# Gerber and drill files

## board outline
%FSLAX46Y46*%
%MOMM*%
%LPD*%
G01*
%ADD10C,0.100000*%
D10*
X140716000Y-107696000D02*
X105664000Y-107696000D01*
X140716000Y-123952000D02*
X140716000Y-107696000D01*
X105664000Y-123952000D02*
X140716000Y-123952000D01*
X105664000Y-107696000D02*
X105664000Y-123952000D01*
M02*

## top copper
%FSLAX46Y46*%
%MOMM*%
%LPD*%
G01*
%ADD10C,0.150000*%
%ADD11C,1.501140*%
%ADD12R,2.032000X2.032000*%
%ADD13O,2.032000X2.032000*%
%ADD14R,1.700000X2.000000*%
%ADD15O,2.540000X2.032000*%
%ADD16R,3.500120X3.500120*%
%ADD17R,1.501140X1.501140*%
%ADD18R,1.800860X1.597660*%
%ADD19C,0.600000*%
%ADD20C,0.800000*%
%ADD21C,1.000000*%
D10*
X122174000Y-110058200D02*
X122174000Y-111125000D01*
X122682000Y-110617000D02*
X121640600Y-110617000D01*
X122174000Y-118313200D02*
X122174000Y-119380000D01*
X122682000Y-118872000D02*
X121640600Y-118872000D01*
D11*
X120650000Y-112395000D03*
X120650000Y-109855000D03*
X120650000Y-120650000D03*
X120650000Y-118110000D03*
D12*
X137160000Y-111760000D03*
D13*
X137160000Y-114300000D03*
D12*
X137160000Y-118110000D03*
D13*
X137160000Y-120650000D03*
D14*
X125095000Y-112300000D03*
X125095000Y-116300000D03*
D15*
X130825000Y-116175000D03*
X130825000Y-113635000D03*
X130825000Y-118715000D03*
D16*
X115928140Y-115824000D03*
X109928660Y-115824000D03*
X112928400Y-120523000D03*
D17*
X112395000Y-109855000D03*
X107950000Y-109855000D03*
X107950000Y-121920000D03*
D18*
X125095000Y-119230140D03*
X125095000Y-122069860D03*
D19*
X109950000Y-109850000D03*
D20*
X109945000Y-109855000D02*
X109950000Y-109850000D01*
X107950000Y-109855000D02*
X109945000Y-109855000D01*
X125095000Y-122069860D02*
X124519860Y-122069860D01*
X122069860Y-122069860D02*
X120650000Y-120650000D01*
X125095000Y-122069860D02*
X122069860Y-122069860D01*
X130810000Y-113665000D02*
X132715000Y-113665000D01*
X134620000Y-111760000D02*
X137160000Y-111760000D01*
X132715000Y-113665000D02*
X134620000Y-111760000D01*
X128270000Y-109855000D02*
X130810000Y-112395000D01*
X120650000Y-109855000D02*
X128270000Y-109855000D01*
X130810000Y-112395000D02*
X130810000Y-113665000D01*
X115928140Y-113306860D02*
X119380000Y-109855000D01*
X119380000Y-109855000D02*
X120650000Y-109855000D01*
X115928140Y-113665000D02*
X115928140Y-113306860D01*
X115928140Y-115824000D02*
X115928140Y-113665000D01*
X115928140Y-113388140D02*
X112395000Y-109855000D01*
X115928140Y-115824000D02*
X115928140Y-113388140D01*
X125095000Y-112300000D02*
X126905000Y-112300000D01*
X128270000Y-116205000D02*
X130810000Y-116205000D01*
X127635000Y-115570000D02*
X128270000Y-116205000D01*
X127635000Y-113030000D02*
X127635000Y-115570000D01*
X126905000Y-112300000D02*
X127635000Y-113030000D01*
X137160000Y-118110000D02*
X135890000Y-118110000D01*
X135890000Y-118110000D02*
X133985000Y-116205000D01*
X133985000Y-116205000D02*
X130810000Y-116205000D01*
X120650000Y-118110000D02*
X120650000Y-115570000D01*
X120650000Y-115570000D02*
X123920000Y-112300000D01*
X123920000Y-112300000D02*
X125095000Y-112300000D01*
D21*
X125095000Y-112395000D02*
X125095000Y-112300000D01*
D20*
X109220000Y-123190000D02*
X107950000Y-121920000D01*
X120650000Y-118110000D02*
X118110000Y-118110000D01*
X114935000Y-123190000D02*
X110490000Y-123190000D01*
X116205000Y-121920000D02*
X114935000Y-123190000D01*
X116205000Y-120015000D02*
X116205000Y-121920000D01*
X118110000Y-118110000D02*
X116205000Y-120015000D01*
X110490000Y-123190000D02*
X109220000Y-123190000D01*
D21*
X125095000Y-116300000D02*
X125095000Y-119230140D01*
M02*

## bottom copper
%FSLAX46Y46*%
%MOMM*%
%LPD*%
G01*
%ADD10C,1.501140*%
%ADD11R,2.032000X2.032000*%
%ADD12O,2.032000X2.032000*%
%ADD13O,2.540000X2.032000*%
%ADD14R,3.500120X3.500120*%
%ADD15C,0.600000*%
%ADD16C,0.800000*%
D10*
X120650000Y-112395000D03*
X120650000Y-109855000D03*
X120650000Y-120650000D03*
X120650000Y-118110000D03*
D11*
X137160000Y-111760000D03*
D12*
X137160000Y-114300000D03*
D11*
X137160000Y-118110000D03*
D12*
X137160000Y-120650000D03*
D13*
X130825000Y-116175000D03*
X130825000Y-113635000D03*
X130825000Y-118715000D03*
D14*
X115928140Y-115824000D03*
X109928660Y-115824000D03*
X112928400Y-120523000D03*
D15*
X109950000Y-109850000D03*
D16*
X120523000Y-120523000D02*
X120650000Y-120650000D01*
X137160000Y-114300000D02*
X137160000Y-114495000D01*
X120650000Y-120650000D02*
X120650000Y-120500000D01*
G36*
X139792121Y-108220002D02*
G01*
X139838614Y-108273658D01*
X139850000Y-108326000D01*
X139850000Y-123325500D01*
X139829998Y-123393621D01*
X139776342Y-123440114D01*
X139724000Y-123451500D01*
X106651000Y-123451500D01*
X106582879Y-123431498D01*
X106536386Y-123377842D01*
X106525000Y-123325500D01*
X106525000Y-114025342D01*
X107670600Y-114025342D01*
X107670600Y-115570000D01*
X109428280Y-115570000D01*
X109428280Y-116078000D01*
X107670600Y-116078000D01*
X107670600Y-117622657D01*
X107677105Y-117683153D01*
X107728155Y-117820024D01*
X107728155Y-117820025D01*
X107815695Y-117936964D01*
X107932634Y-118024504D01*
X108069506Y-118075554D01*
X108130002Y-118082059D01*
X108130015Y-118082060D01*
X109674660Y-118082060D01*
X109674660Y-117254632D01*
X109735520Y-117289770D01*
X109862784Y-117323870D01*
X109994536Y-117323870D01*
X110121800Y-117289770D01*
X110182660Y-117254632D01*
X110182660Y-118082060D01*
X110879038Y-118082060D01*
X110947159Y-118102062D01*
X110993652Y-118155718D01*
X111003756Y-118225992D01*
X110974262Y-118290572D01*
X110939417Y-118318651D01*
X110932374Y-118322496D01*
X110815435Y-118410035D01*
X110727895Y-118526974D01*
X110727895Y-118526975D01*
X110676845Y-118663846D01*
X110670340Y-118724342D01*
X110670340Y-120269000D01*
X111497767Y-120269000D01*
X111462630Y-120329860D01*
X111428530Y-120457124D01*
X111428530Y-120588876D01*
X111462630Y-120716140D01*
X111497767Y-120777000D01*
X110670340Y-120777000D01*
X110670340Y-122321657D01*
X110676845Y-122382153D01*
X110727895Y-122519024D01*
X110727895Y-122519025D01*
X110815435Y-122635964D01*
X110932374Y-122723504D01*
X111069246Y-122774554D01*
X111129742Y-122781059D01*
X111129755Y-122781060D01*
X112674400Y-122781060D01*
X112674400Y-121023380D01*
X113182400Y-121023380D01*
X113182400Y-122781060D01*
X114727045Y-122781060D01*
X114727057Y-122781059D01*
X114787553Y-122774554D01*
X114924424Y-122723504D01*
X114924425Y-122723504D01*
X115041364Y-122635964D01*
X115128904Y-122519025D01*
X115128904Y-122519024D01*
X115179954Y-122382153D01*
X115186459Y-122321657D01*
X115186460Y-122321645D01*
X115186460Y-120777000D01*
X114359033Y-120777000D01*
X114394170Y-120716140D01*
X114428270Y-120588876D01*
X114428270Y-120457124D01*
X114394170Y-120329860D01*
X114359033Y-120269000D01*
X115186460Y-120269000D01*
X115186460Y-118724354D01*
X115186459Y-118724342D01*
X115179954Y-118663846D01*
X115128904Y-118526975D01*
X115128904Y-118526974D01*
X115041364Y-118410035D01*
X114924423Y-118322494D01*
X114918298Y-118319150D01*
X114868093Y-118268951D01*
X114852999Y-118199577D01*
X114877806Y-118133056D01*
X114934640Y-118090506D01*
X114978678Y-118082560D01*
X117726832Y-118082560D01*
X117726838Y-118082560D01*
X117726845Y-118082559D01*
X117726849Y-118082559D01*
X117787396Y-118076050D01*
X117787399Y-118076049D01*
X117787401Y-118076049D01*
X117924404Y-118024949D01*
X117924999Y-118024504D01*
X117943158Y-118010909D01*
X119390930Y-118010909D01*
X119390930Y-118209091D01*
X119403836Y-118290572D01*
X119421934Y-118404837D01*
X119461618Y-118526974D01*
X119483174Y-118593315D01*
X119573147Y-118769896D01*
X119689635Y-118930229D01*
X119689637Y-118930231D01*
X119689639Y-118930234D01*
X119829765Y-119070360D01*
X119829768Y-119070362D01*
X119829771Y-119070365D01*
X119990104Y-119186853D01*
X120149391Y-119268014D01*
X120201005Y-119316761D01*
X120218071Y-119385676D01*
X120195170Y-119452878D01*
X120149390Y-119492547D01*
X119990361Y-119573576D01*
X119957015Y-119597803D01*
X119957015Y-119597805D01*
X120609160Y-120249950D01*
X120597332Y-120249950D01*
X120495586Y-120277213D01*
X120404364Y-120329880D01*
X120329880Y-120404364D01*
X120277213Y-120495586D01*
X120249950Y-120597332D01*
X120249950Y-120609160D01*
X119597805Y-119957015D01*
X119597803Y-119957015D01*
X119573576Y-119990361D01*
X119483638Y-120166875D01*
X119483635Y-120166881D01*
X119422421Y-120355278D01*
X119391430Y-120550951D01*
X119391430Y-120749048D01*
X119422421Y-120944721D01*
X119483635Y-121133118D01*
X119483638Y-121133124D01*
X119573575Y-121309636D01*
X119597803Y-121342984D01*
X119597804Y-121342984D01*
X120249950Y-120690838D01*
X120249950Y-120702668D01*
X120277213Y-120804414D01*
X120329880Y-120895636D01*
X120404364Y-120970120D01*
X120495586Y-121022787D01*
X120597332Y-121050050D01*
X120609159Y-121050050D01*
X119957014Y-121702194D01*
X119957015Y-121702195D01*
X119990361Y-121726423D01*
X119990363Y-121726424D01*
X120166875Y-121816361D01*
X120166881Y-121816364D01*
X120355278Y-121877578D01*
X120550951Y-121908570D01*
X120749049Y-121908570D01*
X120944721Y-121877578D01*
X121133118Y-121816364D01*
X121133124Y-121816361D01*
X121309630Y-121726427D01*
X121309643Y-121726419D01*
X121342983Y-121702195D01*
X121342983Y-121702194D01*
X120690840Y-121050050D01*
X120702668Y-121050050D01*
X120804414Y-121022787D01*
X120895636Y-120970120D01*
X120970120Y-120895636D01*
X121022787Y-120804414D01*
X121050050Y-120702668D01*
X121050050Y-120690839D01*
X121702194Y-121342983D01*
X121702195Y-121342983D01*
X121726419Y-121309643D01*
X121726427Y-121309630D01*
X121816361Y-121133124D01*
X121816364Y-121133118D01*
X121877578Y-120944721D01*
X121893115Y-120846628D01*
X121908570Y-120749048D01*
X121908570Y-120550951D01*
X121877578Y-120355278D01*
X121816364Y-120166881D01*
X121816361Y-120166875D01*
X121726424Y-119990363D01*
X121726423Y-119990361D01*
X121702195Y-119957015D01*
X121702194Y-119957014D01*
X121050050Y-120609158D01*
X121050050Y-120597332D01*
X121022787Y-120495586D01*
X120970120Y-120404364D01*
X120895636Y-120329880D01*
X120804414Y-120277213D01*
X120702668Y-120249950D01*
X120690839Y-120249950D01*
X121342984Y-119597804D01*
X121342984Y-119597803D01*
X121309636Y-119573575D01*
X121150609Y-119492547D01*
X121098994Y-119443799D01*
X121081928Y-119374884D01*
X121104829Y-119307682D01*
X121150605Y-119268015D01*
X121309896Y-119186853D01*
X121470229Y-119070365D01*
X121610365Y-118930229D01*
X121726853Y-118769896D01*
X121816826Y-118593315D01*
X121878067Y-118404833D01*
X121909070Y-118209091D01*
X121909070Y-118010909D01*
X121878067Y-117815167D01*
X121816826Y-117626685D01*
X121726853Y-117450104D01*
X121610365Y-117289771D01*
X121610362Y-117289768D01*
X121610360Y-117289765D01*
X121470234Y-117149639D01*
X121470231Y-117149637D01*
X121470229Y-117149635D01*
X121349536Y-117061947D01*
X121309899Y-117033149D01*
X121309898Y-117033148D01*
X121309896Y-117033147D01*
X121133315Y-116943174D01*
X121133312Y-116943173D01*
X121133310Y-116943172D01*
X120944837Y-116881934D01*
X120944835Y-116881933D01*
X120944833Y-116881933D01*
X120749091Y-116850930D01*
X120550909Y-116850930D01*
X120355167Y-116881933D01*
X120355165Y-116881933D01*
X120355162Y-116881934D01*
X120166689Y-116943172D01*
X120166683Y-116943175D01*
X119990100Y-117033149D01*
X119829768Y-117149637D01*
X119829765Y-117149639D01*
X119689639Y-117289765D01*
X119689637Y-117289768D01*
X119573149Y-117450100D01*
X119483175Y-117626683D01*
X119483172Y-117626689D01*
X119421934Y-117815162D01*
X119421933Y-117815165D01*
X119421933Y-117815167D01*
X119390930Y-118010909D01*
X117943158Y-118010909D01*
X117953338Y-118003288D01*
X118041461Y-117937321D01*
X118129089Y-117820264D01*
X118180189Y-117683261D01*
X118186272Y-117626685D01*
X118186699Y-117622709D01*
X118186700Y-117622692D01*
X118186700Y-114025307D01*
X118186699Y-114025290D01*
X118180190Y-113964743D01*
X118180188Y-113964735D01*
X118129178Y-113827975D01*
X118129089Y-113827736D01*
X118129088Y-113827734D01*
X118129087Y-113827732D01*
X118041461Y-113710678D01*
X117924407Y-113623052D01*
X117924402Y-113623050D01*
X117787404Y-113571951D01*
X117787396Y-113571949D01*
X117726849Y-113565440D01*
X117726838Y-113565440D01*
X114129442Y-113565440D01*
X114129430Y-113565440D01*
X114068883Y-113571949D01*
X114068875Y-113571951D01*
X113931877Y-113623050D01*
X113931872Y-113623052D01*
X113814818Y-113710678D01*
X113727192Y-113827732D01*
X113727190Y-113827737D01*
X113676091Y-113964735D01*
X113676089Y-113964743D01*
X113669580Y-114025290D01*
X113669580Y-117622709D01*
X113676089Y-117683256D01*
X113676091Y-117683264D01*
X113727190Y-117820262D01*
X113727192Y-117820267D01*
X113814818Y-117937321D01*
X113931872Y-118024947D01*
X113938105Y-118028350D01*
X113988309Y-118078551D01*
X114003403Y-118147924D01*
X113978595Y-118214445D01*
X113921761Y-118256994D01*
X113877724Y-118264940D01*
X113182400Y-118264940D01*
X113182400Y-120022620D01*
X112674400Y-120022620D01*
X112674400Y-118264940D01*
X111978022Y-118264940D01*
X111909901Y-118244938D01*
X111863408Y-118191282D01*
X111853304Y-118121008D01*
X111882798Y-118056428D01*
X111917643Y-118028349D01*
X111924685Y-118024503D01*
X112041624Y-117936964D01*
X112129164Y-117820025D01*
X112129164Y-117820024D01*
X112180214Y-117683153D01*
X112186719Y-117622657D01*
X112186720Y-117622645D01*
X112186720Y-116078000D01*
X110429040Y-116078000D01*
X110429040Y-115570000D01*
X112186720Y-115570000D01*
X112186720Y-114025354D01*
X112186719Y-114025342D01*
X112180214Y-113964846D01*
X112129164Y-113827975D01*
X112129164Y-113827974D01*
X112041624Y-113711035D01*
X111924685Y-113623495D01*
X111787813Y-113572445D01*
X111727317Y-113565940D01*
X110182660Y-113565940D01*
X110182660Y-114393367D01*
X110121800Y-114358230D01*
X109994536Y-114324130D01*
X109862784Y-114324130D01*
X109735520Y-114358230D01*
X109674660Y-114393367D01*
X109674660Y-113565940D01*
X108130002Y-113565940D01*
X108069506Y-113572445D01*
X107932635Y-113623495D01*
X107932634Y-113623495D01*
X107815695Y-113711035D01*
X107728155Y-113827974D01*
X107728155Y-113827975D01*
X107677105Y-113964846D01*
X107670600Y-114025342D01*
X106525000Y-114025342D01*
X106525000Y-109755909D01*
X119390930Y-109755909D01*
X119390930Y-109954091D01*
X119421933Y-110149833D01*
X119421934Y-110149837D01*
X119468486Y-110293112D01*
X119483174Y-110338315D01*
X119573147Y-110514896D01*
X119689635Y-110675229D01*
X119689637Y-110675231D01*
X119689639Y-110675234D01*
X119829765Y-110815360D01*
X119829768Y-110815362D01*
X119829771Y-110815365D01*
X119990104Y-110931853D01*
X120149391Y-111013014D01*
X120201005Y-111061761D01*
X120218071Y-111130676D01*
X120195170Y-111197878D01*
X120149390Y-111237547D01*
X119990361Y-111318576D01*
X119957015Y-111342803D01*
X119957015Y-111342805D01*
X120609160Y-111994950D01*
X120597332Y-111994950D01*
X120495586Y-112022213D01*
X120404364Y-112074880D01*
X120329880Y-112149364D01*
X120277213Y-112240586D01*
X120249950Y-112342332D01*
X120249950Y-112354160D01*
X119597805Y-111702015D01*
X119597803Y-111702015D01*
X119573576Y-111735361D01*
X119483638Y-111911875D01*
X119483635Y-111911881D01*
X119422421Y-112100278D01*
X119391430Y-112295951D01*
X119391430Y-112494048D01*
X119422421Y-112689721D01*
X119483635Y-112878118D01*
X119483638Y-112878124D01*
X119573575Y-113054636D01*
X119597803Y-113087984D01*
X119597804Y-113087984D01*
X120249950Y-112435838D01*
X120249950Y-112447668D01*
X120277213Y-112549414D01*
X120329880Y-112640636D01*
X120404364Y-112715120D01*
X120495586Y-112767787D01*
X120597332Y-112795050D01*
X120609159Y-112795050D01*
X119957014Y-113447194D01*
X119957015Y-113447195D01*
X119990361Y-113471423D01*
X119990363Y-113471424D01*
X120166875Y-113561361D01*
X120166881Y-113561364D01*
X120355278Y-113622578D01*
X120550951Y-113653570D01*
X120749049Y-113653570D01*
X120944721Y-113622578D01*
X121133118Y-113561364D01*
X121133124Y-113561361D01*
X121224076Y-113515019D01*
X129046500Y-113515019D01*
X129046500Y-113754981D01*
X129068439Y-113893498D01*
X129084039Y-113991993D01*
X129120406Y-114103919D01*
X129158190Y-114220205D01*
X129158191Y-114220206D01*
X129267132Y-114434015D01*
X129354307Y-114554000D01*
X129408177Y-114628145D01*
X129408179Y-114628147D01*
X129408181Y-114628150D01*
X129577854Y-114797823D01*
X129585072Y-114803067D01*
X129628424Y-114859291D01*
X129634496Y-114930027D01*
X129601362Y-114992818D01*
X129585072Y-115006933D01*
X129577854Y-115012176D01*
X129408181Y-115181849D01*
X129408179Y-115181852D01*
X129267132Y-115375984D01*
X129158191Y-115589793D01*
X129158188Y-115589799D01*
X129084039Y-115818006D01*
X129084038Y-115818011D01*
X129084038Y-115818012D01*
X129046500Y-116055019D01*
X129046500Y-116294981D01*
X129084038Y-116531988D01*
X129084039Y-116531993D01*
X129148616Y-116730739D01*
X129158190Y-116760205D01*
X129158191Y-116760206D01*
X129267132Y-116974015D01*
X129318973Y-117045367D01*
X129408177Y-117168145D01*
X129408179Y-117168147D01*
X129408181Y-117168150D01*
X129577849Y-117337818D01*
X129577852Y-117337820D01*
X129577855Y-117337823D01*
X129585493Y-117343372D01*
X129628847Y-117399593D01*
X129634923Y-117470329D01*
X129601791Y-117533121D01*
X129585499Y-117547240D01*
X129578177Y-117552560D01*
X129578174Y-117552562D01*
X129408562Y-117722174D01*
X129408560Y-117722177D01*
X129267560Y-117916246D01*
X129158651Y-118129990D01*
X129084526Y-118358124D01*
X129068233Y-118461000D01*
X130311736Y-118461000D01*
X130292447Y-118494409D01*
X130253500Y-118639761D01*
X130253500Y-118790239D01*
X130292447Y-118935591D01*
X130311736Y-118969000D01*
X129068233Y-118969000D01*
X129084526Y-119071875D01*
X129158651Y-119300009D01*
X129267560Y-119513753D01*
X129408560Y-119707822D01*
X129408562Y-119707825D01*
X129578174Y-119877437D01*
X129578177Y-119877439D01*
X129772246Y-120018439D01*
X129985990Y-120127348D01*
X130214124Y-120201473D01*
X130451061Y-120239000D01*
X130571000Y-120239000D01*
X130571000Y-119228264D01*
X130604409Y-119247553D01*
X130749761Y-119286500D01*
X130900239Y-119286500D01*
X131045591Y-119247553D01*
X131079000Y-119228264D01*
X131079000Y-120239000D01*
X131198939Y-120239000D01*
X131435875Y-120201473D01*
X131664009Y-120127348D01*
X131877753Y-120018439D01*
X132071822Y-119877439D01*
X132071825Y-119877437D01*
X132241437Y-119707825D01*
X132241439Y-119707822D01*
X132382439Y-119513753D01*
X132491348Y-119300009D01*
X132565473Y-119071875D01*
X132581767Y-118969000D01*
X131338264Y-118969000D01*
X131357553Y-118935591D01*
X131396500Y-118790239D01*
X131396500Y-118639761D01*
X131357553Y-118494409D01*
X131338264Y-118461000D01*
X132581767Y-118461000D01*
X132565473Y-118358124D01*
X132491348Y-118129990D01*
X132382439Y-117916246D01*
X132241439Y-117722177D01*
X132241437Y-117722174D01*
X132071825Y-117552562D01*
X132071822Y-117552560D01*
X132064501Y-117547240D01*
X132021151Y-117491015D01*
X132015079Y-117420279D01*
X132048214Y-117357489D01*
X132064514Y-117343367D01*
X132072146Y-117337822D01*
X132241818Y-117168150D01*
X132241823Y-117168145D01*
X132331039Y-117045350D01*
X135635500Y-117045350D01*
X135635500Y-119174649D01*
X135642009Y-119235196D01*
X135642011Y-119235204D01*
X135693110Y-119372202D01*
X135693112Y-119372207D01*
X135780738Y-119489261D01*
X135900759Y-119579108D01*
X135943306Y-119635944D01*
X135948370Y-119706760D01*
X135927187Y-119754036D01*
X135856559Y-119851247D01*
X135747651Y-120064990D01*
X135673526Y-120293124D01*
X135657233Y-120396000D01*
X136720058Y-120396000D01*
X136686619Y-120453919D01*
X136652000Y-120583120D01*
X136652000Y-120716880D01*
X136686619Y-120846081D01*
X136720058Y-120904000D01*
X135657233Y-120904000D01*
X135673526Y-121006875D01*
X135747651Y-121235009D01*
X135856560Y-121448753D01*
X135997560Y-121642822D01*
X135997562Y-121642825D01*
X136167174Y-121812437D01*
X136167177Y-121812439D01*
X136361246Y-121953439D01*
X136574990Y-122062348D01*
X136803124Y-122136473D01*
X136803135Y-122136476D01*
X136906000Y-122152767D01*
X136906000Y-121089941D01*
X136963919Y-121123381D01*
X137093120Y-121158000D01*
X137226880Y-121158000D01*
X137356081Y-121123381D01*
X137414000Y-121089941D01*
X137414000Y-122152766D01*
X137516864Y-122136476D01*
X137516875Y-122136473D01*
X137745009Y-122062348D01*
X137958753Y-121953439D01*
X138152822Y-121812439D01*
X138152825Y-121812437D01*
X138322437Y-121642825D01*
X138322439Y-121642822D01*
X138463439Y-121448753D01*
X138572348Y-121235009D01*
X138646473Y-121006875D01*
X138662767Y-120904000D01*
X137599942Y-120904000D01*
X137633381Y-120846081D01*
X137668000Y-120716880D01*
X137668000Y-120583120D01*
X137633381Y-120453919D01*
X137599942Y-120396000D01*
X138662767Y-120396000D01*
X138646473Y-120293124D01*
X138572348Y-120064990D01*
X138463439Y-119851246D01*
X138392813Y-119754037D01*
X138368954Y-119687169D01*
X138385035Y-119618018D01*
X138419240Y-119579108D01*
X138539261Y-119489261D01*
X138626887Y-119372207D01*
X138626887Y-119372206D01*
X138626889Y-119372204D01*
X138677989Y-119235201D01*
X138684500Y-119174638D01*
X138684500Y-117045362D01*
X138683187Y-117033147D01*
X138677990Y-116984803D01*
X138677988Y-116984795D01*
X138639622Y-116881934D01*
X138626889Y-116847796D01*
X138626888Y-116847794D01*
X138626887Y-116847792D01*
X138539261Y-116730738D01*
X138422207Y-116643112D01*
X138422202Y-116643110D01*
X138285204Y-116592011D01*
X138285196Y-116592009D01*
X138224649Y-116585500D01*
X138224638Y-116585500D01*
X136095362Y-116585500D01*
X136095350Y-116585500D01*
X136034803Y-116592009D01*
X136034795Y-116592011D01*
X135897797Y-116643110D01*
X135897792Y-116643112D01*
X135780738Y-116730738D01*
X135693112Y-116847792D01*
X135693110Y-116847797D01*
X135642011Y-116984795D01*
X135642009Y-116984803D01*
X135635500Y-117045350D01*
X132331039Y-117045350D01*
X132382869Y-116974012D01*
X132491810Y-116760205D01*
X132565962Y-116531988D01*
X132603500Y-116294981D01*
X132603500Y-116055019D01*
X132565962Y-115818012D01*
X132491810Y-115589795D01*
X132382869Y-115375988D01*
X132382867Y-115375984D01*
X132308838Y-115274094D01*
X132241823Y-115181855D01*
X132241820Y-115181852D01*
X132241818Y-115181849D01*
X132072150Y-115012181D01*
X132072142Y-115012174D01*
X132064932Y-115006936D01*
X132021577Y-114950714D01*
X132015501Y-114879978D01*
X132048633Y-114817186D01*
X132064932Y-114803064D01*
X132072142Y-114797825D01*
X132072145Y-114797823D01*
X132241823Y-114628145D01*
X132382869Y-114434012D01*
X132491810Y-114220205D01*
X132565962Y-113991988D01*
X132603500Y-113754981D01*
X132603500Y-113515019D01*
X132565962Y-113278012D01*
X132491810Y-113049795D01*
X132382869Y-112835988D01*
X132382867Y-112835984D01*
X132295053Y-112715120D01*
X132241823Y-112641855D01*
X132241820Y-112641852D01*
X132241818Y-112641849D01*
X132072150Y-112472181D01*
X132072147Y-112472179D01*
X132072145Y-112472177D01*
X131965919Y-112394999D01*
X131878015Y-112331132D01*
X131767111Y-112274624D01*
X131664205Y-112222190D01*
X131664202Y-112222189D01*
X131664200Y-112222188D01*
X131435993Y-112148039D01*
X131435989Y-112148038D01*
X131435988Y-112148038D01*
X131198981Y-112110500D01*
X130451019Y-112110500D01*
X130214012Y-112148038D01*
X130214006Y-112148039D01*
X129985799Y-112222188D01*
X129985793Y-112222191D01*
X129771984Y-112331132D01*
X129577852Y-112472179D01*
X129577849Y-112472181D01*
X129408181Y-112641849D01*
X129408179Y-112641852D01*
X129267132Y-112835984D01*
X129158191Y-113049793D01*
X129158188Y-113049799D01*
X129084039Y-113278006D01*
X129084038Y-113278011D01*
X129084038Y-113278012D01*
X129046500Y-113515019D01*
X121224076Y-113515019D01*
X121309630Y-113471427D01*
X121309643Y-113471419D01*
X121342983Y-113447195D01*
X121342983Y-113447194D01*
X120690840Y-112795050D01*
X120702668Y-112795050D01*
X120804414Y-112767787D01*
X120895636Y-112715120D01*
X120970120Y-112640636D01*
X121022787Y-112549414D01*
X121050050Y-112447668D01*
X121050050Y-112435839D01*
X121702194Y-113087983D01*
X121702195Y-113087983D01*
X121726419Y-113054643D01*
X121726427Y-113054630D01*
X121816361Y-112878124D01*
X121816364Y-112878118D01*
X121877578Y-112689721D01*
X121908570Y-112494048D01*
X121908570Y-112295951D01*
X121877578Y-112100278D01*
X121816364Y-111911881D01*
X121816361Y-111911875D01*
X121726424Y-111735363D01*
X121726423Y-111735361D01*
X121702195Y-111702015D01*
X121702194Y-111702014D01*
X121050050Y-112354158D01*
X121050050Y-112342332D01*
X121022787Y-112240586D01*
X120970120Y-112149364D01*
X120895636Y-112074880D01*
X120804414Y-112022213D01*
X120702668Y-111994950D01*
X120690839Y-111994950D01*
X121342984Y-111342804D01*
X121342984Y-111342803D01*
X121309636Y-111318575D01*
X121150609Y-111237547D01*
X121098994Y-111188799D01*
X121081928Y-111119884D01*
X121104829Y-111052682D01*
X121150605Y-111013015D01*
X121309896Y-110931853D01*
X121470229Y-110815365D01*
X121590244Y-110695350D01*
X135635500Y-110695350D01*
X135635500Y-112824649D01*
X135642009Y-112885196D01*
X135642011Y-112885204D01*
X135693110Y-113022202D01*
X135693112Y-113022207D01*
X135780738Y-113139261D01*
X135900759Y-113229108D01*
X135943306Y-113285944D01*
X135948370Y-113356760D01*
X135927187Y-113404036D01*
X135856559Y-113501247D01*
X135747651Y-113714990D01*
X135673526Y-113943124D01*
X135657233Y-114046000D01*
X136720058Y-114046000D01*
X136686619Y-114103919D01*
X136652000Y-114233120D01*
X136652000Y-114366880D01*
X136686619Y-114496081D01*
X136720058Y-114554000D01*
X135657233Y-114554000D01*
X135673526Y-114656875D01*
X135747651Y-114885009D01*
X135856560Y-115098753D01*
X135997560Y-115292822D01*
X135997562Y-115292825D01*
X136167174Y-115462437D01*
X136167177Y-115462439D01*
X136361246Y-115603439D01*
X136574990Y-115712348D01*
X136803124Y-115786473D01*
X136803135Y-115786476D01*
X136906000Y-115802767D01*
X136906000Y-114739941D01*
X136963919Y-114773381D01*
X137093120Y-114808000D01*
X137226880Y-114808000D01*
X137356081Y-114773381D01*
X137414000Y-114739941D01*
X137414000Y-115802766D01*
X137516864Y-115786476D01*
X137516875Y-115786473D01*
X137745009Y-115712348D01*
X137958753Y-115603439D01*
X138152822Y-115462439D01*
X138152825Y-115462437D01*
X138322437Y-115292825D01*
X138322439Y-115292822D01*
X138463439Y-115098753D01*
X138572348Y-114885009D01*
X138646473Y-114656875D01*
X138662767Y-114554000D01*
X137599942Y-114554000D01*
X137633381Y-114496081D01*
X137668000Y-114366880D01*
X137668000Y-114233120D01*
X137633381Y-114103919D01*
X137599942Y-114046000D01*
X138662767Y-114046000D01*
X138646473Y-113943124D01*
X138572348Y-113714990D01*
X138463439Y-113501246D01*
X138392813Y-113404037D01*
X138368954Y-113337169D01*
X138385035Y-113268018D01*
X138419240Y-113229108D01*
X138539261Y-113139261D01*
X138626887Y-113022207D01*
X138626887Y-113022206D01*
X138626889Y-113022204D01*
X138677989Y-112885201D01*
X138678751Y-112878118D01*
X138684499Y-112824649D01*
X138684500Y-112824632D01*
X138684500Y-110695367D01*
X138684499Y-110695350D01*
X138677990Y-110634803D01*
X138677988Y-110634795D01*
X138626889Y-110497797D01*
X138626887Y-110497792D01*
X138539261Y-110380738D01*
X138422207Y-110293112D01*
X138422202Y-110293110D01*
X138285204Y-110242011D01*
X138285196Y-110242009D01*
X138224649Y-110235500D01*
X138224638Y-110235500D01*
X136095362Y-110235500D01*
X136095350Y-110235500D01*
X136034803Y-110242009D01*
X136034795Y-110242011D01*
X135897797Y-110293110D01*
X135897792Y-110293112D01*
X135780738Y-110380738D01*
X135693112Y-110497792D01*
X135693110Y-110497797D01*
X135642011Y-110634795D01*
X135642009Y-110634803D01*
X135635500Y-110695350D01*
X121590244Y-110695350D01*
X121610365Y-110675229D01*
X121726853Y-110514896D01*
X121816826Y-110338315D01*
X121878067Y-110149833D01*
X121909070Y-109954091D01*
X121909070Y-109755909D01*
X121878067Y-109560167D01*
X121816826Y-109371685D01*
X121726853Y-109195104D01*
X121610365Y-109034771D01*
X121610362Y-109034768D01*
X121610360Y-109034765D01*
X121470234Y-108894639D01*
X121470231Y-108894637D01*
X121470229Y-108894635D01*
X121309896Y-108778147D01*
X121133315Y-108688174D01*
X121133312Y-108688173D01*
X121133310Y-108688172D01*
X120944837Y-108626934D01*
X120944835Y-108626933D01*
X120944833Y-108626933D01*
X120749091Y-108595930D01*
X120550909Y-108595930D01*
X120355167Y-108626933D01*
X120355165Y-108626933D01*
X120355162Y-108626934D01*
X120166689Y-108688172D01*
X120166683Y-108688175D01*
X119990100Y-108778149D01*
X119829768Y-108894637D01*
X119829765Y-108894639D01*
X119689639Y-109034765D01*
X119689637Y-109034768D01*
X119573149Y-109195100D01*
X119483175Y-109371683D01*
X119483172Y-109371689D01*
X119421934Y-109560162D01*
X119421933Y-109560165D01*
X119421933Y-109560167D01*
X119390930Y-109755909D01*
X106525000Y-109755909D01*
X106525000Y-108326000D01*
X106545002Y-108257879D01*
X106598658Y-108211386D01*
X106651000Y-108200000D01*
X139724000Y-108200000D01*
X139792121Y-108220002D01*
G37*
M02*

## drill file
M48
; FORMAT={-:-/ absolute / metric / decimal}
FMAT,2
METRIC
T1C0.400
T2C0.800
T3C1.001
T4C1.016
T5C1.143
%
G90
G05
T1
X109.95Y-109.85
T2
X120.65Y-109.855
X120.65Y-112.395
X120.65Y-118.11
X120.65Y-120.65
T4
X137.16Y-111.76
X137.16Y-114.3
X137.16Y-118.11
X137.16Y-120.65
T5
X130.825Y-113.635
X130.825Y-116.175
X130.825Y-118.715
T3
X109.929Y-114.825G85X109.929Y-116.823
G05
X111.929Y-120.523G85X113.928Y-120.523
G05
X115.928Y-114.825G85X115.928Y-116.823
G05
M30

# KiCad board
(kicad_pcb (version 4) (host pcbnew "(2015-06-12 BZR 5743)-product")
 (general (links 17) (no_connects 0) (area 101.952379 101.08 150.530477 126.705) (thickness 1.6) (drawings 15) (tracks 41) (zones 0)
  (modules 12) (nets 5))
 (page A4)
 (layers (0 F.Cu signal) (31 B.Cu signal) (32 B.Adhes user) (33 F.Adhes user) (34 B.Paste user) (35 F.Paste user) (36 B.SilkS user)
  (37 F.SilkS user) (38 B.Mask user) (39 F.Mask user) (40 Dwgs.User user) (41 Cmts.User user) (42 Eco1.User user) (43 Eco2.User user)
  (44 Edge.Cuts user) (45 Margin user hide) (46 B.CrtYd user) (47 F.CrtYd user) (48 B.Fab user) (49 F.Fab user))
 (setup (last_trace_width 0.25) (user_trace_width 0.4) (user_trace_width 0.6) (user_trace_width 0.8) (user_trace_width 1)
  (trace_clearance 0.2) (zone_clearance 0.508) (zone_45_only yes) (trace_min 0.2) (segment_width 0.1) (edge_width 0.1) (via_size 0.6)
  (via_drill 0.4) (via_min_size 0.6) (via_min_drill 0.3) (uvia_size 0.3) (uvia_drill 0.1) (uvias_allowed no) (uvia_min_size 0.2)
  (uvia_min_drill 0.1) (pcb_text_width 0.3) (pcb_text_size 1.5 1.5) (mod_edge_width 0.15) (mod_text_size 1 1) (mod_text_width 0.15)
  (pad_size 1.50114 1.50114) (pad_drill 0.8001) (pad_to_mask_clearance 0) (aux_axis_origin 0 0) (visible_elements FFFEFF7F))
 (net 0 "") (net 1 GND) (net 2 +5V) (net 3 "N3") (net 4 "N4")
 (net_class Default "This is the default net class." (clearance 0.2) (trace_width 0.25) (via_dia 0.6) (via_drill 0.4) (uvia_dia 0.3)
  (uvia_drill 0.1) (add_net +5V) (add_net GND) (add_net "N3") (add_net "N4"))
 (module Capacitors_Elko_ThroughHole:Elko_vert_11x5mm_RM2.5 (layer F.Cu) (at 120.65 109.855 270)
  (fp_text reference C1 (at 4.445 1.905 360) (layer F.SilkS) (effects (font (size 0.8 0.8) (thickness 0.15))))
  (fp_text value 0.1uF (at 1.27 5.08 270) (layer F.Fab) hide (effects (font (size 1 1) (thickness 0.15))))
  (fp_line (start 0.2032 -1.524) (end 1.27 -1.524) (layer F.Cu) (width 0.15))
  (fp_line (start 0.762 -2.032) (end 0.762 -0.9906) (layer F.Cu) (width 0.15))
  (pad 2 thru_hole circle (at 2.54 0 270) (size 1.50114 1.50114) (drill 0.8001) (layers *.Cu *.Mask F.SilkS) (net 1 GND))
  (pad 1 thru_hole circle (at 0 0 270) (size 1.50114 1.50114) (drill 0.8001) (layers *.Cu *.Mask F.SilkS) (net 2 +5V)))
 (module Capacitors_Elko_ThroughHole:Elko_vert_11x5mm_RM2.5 (layer F.Cu) (at 120.65 118.11 270)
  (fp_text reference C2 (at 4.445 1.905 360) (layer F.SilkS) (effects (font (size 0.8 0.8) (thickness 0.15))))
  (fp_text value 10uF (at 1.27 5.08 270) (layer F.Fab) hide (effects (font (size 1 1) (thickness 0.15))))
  (fp_line (start 0.2032 -1.524) (end 1.27 -1.524) (layer F.Cu) (width 0.15))
  (fp_line (start 0.762 -2.032) (end 0.762 -0.9906) (layer F.Cu) (width 0.15))
  (pad 2 thru_hole circle (at 2.54 0 270) (size 1.50114 1.50114) (drill 0.8001) (layers *.Cu *.Mask F.SilkS) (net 1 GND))
  (pad 1 thru_hole circle (at 0 0 270) (size 1.50114 1.50114) (drill 0.8001) (layers *.Cu *.Mask F.SilkS) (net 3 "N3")))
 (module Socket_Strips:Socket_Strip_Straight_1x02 (layer F.Cu) (at 137.16 111.76 270)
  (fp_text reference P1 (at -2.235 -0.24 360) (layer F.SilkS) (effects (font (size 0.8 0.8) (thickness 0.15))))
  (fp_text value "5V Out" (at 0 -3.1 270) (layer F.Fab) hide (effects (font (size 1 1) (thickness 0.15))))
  (pad 1 thru_hole rect (at 0 0 270) (size 2.032 2.032) (drill 1.016) (layers *.Cu *.Mask F.SilkS) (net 2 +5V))
  (pad 2 thru_hole oval (at 2.54 0 270) (size 2.032 2.032) (drill 1.016) (layers *.Cu *.Mask F.SilkS) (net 1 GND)))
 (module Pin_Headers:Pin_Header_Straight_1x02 (layer B.Cu) (at 137.16 118.11 180)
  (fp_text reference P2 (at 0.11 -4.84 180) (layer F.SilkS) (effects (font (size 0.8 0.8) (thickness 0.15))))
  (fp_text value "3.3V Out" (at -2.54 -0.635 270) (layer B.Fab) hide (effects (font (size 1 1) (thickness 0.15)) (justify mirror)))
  (pad 1 thru_hole rect (at 0 0 180) (size 2.032 2.032) (drill 1.016) (layers *.Cu *.Mask B.SilkS) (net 3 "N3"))
  (pad 2 thru_hole oval (at 0 -2.54 180) (size 2.032 2.032) (drill 1.016) (layers *.Cu *.Mask B.SilkS) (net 1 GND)))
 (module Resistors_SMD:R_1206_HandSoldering (layer F.Cu) (at 125.095 114.3 270)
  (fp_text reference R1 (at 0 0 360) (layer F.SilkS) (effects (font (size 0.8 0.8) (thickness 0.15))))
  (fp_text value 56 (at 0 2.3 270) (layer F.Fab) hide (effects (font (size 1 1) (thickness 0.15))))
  (pad 1 smd rect (at -2 0 270) (size 2 1.7) (layers F.Cu F.Paste F.Mask) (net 3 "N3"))
  (pad 2 smd rect (at 2 0 270) (size 2 1.7) (layers F.Cu F.Paste F.Mask) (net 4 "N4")))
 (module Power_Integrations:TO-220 (layer F.Cu) (at 130.825 116.175 90)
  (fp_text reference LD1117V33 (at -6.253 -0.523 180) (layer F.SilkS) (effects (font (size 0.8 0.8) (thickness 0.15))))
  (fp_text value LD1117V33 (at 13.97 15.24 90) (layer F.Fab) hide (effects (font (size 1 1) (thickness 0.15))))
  (pad 2 thru_hole oval (at 0 0 90) (size 2.032 2.54) (drill 1.143) (layers *.Cu *.Mask F.SilkS) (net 3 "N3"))
  (pad 3 thru_hole oval (at 2.54 0 90) (size 2.032 2.54) (drill 1.143) (layers *.Cu *.Mask F.SilkS) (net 2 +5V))
  (pad 1 thru_hole oval (at -2.54 0 90) (size 2.032 2.54) (drill 1.143) (layers *.Cu *.Mask F.SilkS) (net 1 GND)))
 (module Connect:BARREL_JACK (layer F.Cu) (at 109.728 115.824)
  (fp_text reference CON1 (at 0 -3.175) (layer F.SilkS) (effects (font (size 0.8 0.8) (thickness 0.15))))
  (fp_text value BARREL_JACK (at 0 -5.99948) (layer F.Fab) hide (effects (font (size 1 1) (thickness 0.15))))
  (pad 1 thru_hole rect (at 6.20014 0) (size 3.50012 3.50012) (drill oval 1.00076 2.99974) (layers *.Cu *.Mask F.SilkS) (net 2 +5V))
  (pad 2 thru_hole rect (at 0.20066 0) (size 3.50012 3.50012) (drill oval 1.00076 2.99974) (layers *.Cu *.Mask F.SilkS) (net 1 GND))
  (pad 3 thru_hole rect (at 3.2004 4.699) (size 3.50012 3.50012) (drill oval 2.99974 1.00076) (layers *.Cu *.Mask F.SilkS) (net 1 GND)))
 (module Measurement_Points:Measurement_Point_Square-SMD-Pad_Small (layer F.Cu) (at 112.395 109.855)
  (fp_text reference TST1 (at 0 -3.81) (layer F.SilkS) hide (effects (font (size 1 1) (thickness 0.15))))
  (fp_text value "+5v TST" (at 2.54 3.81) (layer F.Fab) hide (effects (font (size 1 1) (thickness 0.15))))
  (pad 1 smd rect (at 0 0) (size 1.50114 1.50114) (layers F.Cu F.Paste F.Mask) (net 2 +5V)))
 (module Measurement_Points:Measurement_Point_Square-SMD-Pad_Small (layer F.Cu) (at 107.95 109.855)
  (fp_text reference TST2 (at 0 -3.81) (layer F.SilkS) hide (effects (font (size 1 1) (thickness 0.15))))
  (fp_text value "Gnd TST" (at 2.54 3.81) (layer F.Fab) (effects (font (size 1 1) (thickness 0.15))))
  (pad 1 smd rect (at 0 0) (size 1.50114 1.50114) (layers F.Cu F.Paste F.Mask) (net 1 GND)))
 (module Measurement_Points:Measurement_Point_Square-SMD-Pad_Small (layer F.Cu) (at 107.95 121.92)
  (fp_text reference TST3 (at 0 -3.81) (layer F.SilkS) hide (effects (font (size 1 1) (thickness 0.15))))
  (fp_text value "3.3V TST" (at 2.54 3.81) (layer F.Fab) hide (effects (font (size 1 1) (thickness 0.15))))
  (pad 1 smd rect (at 0 0) (size 1.50114 1.50114) (layers F.Cu F.Paste F.Mask) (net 3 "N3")))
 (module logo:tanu (layer B.Cu) (at 125.3 115.75 90)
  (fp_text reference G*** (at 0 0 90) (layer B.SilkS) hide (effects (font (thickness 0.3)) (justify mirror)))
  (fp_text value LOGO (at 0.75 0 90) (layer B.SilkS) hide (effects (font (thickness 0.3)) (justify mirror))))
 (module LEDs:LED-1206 (layer F.Cu) (at 125.095 120.65 90)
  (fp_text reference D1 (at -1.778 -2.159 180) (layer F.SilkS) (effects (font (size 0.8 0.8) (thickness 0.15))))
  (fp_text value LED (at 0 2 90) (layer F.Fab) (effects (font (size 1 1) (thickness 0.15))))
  (pad 2 smd rect (at 1.41986 0 270) (size 1.59766 1.80086) (layers F.Cu F.Paste F.Mask) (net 4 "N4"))
  (pad 1 smd rect (at -1.41986 0 270) (size 1.59766 1.80086) (layers F.Cu F.Paste F.Mask) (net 1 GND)))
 (gr_line (start 140.716 107.696) (end 105.664 107.696) (angle 90) (layer Edge.Cuts) (width 0.1))
 (gr_line (start 140.716 123.952) (end 140.716 107.696) (angle 90) (layer Edge.Cuts) (width 0.1))
 (gr_line (start 105.664 123.952) (end 140.716 123.952) (angle 90) (layer Edge.Cuts) (width 0.1))
 (gr_line (start 105.664 107.696) (end 105.664 123.952) (angle 90) (layer Edge.Cuts) (width 0.1))
 (segment (start 120.523 120.523) (end 120.65 120.65) (width 0.8) (layer B.Cu) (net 1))
 (segment (start 137.16 114.3) (end 137.16 114.495) (width 0.8) (layer B.Cu) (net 1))
 (segment (start 120.65 120.65) (end 120.65 120.5) (width 0.8) (layer B.Cu) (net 1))
 (segment (start 109.945 109.855) (end 109.95 109.85) (width 0.8) (layer F.Cu) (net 1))
 (via (at 109.95 109.85) (size 0.6) (layers F.Cu B.Cu) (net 1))
 (segment (start 107.95 109.855) (end 109.945 109.855) (width 0.8) (layer F.Cu) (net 1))
 (segment (start 125.095 122.06986) (end 124.51986 122.06986) (width 0.8) (layer F.Cu) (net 1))
 (segment (start 122.06986 122.06986) (end 120.65 120.65) (width 0.8) (layer F.Cu) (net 1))
 (segment (start 125.095 122.06986) (end 122.06986 122.06986) (width 0.8) (layer F.Cu) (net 1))
 (segment (start 130.81 113.665) (end 132.715 113.665) (width 0.8) (layer F.Cu) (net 2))
 (segment (start 134.62 111.76) (end 137.16 111.76) (width 0.8) (layer F.Cu) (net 2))
 (segment (start 132.715 113.665) (end 134.62 111.76) (width 0.8) (layer F.Cu) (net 2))
 (segment (start 128.27 109.855) (end 130.81 112.395) (width 0.8) (layer F.Cu) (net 2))
 (segment (start 120.65 109.855) (end 128.27 109.855) (width 0.8) (layer F.Cu) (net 2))
 (segment (start 130.81 112.395) (end 130.81 113.665) (width 0.8) (layer F.Cu) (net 2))
 (segment (start 115.92814 113.30686) (end 119.38 109.855) (width 0.8) (layer F.Cu) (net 2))
 (segment (start 119.38 109.855) (end 120.65 109.855) (width 0.8) (layer F.Cu) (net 2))
 (segment (start 115.92814 113.665) (end 115.92814 113.30686) (width 0.8) (layer F.Cu) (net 2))
 (segment (start 115.92814 115.824) (end 115.92814 113.665) (width 0.8) (layer F.Cu) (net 2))
 (segment (start 115.92814 113.38814) (end 112.395 109.855) (width 0.8) (layer F.Cu) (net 2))
 (segment (start 115.92814 115.824) (end 115.92814 113.38814) (width 0.8) (layer F.Cu) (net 2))
 (segment (start 125.095 112.3) (end 126.905 112.3) (width 0.8) (layer F.Cu) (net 3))
 (segment (start 128.27 116.205) (end 130.81 116.205) (width 0.8) (layer F.Cu) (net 3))
 (segment (start 127.635 115.57) (end 128.27 116.205) (width 0.8) (layer F.Cu) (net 3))
 (segment (start 127.635 113.03) (end 127.635 115.57) (width 0.8) (layer F.Cu) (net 3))
 (segment (start 126.905 112.3) (end 127.635 113.03) (width 0.8) (layer F.Cu) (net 3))
 (segment (start 137.16 118.11) (end 135.89 118.11) (width 0.8) (layer F.Cu) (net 3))
 (segment (start 135.89 118.11) (end 133.985 116.205) (width 0.8) (layer F.Cu) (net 3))
 (segment (start 133.985 116.205) (end 130.81 116.205) (width 0.8) (layer F.Cu) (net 3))
 (segment (start 120.65 118.11) (end 120.65 115.57) (width 0.8) (layer F.Cu) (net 3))
 (segment (start 120.65 115.57) (end 123.92 112.3) (width 0.8) (layer F.Cu) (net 3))
 (segment (start 123.92 112.3) (end 125.095 112.3) (width 0.8) (layer F.Cu) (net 3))
 (segment (start 125.095 112.395) (end 125.095 112.3) (width 1) (layer F.Cu) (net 3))
 (segment (start 109.22 123.19) (end 107.95 121.92) (width 0.8) (layer F.Cu) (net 3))
 (segment (start 120.65 118.11) (end 118.11 118.11) (width 0.8) (layer F.Cu) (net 3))
 (segment (start 114.935 123.19) (end 110.49 123.19) (width 0.8) (layer F.Cu) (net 3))
 (segment (start 116.205 121.92) (end 114.935 123.19) (width 0.8) (layer F.Cu) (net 3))
 (segment (start 116.205 120.015) (end 116.205 121.92) (width 0.8) (layer F.Cu) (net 3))
 (segment (start 118.11 118.11) (end 116.205 120.015) (width 0.8) (layer F.Cu) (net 3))
 (segment (start 110.49 123.19) (end 109.22 123.19) (width 0.8) (layer F.Cu) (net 3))
 (segment (start 125.095 116.3) (end 125.095 119.23014) (width 1) (layer F.Cu) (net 4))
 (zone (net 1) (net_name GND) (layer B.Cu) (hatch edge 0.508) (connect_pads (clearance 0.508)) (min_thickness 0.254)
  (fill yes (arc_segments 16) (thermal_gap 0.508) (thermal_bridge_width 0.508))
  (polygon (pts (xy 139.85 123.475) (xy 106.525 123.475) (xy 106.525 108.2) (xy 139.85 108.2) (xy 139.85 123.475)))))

